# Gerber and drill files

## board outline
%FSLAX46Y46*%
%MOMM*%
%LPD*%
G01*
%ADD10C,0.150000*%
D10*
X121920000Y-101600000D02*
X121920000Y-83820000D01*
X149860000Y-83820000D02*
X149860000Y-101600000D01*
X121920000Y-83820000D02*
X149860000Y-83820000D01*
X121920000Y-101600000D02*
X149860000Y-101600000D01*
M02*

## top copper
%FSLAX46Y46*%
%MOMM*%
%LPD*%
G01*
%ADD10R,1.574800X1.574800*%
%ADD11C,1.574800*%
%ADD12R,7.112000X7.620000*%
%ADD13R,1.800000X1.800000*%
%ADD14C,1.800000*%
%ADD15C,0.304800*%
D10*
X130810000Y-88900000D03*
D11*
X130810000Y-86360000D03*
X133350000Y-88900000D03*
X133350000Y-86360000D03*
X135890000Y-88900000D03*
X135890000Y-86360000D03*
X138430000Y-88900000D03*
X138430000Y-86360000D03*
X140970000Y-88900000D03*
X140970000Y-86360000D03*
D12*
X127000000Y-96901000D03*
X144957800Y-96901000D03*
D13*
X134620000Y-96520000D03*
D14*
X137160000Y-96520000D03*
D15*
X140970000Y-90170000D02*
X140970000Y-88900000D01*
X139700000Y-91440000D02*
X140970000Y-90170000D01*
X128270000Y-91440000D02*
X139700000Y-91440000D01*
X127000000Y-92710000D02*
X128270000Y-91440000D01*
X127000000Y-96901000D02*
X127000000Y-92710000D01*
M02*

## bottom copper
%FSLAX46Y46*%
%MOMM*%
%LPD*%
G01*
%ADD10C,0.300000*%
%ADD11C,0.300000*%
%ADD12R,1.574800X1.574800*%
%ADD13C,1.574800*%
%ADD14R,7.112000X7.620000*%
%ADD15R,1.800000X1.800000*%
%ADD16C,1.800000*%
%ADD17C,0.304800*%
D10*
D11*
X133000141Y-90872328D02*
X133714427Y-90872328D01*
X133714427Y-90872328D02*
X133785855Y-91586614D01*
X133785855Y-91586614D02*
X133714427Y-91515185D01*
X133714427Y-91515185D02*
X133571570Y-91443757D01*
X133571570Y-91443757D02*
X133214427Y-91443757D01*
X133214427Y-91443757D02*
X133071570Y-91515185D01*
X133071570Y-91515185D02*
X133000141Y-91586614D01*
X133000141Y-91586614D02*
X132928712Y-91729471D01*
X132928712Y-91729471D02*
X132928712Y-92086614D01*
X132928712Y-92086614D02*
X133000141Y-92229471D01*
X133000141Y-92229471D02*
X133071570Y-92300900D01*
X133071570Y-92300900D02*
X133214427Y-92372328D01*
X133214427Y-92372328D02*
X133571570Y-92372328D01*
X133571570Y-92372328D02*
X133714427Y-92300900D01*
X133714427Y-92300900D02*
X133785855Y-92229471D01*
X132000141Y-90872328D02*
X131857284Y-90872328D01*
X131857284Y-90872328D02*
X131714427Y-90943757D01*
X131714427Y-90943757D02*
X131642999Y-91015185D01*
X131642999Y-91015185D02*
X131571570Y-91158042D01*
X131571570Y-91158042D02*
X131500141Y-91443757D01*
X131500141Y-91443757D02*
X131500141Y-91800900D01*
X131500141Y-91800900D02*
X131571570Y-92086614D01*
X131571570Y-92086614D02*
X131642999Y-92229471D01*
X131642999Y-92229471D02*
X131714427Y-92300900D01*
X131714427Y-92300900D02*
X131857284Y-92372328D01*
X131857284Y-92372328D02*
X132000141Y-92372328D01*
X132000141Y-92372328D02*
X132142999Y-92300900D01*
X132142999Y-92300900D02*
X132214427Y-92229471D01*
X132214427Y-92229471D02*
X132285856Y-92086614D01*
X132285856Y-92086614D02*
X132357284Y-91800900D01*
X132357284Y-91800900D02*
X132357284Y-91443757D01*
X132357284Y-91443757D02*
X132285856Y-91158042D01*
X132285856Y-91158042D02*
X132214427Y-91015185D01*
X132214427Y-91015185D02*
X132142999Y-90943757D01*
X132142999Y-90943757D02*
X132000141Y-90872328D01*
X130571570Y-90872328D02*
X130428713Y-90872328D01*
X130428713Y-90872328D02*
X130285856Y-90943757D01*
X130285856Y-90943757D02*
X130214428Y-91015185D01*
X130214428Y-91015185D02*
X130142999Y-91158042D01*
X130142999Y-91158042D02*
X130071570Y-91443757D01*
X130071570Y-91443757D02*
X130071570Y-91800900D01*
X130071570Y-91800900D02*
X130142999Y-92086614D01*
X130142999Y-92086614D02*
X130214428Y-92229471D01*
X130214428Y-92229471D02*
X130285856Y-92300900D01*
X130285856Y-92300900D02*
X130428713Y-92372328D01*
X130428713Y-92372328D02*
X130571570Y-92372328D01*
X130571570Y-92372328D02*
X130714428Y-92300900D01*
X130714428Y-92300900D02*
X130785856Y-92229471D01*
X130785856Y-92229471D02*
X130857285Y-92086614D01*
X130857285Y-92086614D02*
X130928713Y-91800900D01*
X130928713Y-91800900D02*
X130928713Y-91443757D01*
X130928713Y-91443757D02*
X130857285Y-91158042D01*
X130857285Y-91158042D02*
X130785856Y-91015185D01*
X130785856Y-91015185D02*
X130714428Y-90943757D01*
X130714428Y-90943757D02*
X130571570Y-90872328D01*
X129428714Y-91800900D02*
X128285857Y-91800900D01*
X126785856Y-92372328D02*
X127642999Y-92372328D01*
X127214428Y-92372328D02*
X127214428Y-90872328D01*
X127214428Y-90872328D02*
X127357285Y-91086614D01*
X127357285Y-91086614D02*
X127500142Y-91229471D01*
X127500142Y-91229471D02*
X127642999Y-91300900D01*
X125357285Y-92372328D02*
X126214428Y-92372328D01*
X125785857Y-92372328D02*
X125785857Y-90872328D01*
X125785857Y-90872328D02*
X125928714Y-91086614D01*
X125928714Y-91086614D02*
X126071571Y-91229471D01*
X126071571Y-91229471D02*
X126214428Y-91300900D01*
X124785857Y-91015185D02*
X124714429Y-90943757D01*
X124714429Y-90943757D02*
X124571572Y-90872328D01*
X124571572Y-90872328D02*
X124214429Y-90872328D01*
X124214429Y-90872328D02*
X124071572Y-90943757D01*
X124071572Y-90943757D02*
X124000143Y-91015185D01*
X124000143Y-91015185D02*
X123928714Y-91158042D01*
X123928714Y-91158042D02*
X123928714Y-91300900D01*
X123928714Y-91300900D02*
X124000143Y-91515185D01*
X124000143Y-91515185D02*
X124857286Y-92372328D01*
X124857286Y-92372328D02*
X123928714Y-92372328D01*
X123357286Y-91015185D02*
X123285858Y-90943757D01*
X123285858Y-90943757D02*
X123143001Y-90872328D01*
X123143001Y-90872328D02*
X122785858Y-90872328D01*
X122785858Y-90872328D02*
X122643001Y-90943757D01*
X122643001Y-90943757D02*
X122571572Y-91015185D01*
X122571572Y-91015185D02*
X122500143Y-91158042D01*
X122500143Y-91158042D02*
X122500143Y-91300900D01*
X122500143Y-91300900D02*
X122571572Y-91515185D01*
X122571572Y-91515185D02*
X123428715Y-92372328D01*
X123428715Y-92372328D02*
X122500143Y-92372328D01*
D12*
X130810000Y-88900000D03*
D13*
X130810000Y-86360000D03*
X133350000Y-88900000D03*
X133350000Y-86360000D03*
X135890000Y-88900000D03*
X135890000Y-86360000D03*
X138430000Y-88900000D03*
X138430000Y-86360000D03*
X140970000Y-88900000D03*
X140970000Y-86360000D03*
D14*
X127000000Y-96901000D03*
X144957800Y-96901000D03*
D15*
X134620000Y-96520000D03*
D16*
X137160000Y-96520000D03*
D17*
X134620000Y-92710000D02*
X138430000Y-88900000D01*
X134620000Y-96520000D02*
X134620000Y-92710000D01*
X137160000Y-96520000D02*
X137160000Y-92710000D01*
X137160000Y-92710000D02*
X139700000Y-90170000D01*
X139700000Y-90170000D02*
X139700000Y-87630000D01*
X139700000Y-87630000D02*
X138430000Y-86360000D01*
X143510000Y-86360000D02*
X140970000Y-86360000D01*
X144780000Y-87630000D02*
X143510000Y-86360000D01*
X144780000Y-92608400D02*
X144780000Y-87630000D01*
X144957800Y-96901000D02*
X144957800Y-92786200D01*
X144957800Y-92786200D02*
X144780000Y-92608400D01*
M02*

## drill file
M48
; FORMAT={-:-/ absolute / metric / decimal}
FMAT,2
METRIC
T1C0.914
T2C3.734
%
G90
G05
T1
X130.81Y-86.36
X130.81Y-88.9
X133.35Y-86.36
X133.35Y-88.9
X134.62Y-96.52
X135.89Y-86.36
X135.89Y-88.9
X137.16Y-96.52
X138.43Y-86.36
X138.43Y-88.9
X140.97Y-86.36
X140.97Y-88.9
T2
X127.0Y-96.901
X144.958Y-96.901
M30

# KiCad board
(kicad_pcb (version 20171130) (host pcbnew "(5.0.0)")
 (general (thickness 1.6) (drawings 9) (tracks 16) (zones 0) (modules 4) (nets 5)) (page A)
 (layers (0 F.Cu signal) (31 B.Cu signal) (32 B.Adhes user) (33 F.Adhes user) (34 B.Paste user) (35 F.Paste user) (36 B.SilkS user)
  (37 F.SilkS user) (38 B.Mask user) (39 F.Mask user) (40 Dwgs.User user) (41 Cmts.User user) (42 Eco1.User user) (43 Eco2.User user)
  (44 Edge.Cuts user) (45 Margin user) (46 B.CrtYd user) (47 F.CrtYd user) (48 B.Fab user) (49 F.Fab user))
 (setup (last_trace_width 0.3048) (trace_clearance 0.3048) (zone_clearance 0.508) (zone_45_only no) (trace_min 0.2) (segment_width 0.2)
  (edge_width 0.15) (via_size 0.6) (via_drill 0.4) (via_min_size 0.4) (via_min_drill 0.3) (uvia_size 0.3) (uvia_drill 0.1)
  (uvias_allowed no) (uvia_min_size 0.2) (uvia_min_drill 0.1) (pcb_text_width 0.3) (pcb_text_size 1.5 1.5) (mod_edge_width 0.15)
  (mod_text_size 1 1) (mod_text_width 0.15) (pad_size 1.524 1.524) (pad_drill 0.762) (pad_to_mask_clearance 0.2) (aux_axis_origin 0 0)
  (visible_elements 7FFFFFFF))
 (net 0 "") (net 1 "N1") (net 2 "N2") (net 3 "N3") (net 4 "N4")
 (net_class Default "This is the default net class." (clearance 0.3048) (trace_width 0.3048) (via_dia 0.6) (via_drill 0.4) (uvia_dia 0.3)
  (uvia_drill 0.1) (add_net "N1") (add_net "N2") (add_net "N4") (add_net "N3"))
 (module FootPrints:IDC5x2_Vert (layer F.Cu) (at 135.89 87.63 180)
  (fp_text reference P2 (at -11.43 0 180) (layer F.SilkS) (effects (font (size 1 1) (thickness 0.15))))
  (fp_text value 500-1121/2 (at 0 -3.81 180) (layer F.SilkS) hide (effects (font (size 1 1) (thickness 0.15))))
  (pad 1 thru_hole rect (at 5.08 -1.27 180) (size 1.5748 1.5748) (drill 0.9144) (layers *.Cu *.Mask F.SilkS))
  (pad 2 thru_hole circle (at 5.08 1.27 180) (size 1.5748 1.5748) (drill 0.9144) (layers *.Cu *.Mask F.SilkS))
  (pad 3 thru_hole circle (at 2.54 -1.27 180) (size 1.5748 1.5748) (drill 0.9144) (layers *.Cu *.Mask F.SilkS))
  (pad 4 thru_hole circle (at 2.54 1.27 180) (size 1.5748 1.5748) (drill 0.9144) (layers *.Cu *.Mask F.SilkS))
  (pad 5 thru_hole circle (at 0 -1.27 180) (size 1.5748 1.5748) (drill 0.9144) (layers *.Cu *.Mask F.SilkS))
  (pad 6 thru_hole circle (at 0 1.27 180) (size 1.5748 1.5748) (drill 0.9144) (layers *.Cu *.Mask F.SilkS))
  (pad 7 thru_hole circle (at -2.54 -1.27 180) (size 1.5748 1.5748) (drill 0.9144) (layers *.Cu *.Mask F.SilkS) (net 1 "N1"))
  (pad 8 thru_hole circle (at -2.54 1.27 180) (size 1.5748 1.5748) (drill 0.9144) (layers *.Cu *.Mask F.SilkS) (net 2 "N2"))
  (pad 9 thru_hole circle (at -5.08 -1.27 180) (size 1.5748 1.5748) (drill 0.9144) (layers *.Cu *.Mask F.SilkS) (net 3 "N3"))
  (pad 10 thru_hole circle (at -5.08 1.27 180) (size 1.5748 1.5748) (drill 0.9144) (layers *.Cu *.Mask F.SilkS) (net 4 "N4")))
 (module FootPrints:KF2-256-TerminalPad (layer F.Cu) (at 127 101.6)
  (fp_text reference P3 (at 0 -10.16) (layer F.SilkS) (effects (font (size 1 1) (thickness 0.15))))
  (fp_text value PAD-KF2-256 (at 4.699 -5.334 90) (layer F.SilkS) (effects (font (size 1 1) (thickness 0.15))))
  (pad 1 thru_hole rect (at 0 -4.699) (size 7.112 7.62) (drill 3.7338) (layers *.Cu *.Mask F.SilkS) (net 3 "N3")))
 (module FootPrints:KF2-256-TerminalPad (layer F.Cu) (at 144.9578 101.6)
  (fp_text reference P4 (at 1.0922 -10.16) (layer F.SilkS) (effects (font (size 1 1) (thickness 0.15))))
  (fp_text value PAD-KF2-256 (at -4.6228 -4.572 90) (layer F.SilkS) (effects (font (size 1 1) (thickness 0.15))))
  (pad 1 thru_hole rect (at 0 -4.699) (size 7.112 7.62) (drill 3.7338) (layers *.Cu *.Mask F.SilkS) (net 4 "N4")))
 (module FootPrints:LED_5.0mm (layer F.Cu) (at 134.62 96.52)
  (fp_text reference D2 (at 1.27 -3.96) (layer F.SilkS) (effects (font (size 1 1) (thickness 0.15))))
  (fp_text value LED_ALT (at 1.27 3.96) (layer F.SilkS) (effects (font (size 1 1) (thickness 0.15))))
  (pad 1 thru_hole rect (at 0 0) (size 1.8 1.8) (drill 0.9144) (layers *.Cu *.Mask) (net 1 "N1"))
  (pad 2 thru_hole circle (at 2.54 0) (size 1.8 1.8) (drill 0.9144) (layers *.Cu *.Mask) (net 2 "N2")))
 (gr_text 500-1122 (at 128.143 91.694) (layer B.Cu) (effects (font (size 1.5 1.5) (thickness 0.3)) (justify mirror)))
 (gr_line (start 121.92 101.6) (end 121.92 83.82) (angle 90) (layer Edge.Cuts) (width 0.15))
 (gr_line (start 149.86 83.82) (end 149.86 101.6) (angle 90) (layer Edge.Cuts) (width 0.15))
 (gr_line (start 121.92 83.82) (end 149.86 83.82) (angle 90) (layer Edge.Cuts) (width 0.15))
 (gr_line (start 121.92 101.6) (end 149.86 101.6) (angle 90) (layer Edge.Cuts) (width 0.15))
 (segment (start 134.62 92.71) (end 138.43 88.9) (width 0.3048) (layer B.Cu) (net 1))
 (segment (start 134.62 96.52) (end 134.62 92.71) (width 0.3048) (layer B.Cu) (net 1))
 (segment (start 137.16 96.52) (end 137.16 92.71) (width 0.3048) (layer B.Cu) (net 2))
 (segment (start 137.16 92.71) (end 139.7 90.17) (width 0.3048) (layer B.Cu) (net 2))
 (segment (start 139.7 90.17) (end 139.7 87.63) (width 0.3048) (layer B.Cu) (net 2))
 (segment (start 139.7 87.63) (end 138.43 86.36) (width 0.3048) (layer B.Cu) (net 2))
 (segment (start 140.97 90.17) (end 140.97 88.9) (width 0.3048) (layer F.Cu) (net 3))
 (segment (start 139.7 91.44) (end 140.97 90.17) (width 0.3048) (layer F.Cu) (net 3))
 (segment (start 128.27 91.44) (end 139.7 91.44) (width 0.3048) (layer F.Cu) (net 3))
 (segment (start 127 92.71) (end 128.27 91.44) (width 0.3048) (layer F.Cu) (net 3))
 (segment (start 127 96.901) (end 127 92.71) (width 0.3048) (layer F.Cu) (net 3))
 (segment (start 143.51 86.36) (end 140.97 86.36) (width 0.3048) (layer B.Cu) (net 4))
 (segment (start 144.78 87.63) (end 143.51 86.36) (width 0.3048) (layer B.Cu) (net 4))
 (segment (start 144.78 92.6084) (end 144.78 87.63) (width 0.3048) (layer B.Cu) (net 4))
 (segment (start 144.9578 96.901) (end 144.9578 92.7862) (width 0.3048) (layer B.Cu) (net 4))
 (segment (start 144.9578 92.7862) (end 144.78 92.6084) (width 0.3048) (layer B.Cu) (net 4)))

